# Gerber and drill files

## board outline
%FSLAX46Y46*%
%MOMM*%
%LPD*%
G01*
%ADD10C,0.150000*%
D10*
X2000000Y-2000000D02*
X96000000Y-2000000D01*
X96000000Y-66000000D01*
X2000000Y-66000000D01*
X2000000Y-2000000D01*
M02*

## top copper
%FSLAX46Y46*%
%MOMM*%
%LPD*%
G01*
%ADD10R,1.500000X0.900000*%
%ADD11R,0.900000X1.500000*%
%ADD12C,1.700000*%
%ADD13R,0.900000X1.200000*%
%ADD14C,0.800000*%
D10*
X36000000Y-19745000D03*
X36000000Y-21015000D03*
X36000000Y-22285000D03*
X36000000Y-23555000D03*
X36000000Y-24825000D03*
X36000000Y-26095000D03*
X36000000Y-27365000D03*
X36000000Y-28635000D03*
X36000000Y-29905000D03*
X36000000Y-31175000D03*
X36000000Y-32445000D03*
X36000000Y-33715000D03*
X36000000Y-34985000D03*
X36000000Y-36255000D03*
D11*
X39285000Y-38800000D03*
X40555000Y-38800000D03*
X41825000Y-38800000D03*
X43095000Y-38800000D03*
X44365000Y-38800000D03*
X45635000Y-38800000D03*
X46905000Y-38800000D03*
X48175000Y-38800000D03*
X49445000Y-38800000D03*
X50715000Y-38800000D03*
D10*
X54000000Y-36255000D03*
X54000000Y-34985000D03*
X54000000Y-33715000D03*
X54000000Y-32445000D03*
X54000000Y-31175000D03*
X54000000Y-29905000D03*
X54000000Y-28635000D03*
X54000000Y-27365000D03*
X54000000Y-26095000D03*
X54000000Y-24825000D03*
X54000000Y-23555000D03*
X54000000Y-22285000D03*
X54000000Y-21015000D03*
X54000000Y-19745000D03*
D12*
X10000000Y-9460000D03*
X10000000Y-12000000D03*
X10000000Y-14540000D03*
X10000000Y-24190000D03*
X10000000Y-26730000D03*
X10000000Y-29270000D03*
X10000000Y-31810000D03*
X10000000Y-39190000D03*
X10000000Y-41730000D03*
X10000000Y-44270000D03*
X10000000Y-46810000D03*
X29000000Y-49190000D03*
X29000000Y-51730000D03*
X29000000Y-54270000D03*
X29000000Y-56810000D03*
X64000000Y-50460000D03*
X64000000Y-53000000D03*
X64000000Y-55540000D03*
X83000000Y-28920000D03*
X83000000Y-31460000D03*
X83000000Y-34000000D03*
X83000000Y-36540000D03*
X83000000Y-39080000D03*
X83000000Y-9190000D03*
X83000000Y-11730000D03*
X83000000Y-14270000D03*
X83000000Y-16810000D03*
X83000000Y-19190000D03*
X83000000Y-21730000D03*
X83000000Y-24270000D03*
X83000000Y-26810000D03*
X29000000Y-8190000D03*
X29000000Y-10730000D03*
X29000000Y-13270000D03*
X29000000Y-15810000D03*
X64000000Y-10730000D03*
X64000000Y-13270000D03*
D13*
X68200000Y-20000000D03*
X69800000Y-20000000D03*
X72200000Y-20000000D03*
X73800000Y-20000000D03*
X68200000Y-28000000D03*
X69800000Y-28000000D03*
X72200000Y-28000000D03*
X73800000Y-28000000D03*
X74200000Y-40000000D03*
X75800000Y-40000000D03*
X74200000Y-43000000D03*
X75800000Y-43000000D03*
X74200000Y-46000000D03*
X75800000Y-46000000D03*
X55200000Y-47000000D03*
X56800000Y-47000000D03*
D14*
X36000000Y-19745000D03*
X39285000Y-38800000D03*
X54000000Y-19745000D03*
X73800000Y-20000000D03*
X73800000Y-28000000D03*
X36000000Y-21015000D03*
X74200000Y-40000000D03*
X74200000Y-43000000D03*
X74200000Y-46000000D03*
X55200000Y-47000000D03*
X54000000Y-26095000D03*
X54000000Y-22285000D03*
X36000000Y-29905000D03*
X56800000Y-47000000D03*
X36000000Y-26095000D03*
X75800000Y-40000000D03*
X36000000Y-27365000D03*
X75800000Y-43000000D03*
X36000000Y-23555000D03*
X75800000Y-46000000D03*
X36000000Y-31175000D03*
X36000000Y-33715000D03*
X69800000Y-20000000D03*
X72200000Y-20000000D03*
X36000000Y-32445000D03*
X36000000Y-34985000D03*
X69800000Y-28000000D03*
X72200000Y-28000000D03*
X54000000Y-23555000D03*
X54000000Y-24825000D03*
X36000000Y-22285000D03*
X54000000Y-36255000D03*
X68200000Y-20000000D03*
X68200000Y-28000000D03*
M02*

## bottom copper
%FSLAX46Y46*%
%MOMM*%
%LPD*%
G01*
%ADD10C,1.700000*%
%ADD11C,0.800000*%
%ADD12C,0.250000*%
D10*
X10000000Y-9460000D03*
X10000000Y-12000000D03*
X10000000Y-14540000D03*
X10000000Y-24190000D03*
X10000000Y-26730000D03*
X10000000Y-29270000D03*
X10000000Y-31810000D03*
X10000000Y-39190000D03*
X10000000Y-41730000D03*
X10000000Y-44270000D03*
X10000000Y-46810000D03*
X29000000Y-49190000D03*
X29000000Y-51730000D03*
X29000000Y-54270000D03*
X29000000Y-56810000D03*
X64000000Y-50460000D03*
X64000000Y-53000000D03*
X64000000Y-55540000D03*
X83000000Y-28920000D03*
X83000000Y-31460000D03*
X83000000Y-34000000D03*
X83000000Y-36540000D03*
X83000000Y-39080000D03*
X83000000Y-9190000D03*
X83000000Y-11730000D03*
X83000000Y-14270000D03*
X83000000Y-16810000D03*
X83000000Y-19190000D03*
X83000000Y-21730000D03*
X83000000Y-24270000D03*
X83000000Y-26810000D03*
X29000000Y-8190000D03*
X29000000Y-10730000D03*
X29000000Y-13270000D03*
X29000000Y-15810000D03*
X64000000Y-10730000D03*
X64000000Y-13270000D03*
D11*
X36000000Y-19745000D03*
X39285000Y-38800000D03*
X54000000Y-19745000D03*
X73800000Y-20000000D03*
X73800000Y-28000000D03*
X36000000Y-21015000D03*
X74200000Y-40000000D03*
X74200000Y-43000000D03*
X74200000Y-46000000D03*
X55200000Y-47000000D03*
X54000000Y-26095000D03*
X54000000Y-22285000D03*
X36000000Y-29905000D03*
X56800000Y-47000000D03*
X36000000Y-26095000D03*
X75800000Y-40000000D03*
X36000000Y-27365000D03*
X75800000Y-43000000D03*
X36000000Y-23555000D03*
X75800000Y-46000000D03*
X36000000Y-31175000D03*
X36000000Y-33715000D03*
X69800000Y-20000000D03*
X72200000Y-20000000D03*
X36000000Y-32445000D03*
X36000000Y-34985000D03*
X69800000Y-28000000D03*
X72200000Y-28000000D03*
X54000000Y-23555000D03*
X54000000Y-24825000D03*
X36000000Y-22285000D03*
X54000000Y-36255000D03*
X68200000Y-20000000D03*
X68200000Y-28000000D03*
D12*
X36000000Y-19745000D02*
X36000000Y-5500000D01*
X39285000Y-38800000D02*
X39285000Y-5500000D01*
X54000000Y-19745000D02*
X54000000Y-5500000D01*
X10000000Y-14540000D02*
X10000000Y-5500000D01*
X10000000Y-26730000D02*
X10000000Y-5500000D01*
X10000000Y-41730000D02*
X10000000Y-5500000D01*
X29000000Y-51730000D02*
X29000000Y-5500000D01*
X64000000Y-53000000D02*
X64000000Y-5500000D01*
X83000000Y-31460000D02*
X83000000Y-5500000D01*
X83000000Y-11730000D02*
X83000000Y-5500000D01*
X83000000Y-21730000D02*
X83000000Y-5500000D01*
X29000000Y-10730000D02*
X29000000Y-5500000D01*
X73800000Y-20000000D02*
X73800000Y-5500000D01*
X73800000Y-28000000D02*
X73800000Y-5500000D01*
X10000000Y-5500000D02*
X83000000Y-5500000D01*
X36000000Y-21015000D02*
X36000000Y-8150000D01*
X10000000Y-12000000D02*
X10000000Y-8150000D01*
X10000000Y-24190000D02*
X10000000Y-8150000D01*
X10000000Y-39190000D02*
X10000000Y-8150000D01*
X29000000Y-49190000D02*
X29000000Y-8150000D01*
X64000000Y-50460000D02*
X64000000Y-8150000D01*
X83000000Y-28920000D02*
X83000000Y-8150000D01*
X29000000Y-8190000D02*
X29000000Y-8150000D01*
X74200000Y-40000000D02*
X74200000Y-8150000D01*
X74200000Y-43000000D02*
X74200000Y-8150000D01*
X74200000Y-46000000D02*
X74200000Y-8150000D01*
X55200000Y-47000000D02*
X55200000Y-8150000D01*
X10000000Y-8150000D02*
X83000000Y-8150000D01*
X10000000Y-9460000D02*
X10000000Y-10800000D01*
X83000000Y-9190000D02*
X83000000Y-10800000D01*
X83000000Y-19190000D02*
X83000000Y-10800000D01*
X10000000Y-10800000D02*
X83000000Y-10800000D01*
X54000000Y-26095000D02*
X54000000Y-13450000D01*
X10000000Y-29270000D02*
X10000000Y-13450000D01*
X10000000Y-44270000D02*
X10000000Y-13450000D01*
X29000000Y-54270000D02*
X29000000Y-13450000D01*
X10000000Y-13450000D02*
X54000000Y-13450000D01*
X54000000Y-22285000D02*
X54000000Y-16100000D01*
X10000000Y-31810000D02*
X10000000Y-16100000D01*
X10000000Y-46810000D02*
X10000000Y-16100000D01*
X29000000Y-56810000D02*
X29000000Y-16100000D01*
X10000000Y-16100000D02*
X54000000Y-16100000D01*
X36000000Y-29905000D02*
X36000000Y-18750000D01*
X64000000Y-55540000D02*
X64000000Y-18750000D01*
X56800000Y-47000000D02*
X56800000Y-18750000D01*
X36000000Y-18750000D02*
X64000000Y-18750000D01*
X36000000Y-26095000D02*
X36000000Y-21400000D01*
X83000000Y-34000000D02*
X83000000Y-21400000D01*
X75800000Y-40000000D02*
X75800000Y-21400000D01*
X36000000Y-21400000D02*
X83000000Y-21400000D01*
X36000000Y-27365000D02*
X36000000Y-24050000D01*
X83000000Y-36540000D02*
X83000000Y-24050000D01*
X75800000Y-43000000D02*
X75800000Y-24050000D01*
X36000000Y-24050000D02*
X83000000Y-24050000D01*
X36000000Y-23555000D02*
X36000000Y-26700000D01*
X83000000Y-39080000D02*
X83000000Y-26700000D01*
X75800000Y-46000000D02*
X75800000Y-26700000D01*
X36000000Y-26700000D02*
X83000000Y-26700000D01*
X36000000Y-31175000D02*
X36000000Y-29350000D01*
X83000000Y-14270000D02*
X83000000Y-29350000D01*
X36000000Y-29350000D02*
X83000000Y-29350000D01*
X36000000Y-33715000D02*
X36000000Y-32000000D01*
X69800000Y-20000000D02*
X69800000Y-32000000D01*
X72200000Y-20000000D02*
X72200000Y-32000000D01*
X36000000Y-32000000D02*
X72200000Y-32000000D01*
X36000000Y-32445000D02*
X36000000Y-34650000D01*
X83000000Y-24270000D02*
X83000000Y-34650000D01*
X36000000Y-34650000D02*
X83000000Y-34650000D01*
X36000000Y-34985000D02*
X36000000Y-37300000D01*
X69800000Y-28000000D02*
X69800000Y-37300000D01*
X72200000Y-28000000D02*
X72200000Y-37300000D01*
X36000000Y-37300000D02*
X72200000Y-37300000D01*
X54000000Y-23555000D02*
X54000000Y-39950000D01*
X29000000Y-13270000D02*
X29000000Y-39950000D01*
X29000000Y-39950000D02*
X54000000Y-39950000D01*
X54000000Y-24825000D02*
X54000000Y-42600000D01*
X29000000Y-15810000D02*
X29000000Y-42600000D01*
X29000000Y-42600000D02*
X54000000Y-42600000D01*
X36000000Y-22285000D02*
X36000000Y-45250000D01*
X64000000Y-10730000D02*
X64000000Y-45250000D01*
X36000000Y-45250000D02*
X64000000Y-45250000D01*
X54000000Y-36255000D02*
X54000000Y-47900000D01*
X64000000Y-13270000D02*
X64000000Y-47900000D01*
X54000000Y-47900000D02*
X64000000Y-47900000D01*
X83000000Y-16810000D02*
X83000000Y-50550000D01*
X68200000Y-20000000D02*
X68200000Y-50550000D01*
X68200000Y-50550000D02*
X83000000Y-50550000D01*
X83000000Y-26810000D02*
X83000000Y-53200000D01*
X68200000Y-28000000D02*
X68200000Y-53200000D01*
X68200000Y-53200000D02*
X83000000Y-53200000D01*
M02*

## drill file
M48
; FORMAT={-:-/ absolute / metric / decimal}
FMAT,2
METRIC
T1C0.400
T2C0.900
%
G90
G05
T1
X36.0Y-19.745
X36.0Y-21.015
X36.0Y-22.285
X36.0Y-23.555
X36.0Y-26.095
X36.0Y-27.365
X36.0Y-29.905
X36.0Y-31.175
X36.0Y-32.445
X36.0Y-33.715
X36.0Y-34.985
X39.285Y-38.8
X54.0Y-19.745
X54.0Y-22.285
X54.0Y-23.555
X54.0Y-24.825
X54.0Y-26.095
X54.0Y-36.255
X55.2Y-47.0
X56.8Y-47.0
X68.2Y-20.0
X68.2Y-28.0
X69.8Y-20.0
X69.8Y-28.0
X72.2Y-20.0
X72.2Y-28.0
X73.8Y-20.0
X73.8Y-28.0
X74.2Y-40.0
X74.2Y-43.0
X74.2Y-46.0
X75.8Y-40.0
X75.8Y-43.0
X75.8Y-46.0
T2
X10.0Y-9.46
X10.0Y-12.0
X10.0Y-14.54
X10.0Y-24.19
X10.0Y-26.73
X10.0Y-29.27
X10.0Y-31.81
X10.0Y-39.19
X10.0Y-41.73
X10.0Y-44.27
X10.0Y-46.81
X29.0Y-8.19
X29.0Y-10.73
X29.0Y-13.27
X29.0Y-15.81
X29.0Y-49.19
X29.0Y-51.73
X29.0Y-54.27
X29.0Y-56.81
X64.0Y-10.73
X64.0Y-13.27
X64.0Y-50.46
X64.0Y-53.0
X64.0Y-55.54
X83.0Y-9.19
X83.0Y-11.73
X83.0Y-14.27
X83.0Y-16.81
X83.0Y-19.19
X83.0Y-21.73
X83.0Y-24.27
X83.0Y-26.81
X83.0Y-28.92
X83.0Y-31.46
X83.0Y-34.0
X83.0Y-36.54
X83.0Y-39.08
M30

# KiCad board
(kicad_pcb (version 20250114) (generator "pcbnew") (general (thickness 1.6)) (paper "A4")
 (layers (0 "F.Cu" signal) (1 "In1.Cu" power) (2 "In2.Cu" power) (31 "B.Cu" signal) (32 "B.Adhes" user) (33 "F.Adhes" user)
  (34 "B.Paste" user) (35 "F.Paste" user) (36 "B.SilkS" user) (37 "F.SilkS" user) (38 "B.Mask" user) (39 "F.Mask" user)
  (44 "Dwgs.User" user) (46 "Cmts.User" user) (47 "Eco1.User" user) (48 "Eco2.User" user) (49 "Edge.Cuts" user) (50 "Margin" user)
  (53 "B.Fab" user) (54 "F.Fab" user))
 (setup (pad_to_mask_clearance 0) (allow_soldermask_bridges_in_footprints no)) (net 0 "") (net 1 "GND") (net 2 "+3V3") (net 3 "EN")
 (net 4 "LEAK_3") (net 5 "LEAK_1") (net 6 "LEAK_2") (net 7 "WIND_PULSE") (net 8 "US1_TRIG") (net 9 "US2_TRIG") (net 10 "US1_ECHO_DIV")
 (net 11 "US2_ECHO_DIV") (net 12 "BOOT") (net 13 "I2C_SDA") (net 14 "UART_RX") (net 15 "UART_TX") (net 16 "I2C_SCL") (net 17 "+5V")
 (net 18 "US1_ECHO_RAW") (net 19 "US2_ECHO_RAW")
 (gr_rect (start 2 2) (end 96 66) (stroke (width 0.15) (type default)) (fill none) (layer "Edge.Cuts"))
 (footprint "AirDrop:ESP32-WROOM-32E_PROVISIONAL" (layer "F.Cu") (at 45 28)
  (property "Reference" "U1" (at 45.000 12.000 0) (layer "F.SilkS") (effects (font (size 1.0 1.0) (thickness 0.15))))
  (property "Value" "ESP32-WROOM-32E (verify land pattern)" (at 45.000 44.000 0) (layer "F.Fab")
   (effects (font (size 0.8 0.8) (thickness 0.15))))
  (pad "1" smd rect (at -9.000 -8.255) (size 1.5 0.9) (layers "F.Cu" "F.Paste" "F.Mask") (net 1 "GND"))
  (pad "2" smd rect (at -9.000 -6.985) (size 1.5 0.9) (layers "F.Cu" "F.Paste" "F.Mask") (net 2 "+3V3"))
  (pad "3" smd rect (at -9.000 -5.715) (size 1.5 0.9) (layers "F.Cu" "F.Paste" "F.Mask") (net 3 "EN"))
  (pad "4" smd rect (at -9.000 -4.445) (size 1.5 0.9) (layers "F.Cu" "F.Paste" "F.Mask") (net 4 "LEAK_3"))
  (pad "5" smd rect (at -9.000 -3.175) (size 1.5 0.9) (layers "F.Cu" "F.Paste" "F.Mask"))
  (pad "6" smd rect (at -9.000 -1.905) (size 1.5 0.9) (layers "F.Cu" "F.Paste" "F.Mask") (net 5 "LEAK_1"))
  (pad "7" smd rect (at -9.000 -0.635) (size 1.5 0.9) (layers "F.Cu" "F.Paste" "F.Mask") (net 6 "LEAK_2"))
  (pad "8" smd rect (at -9.000 0.635) (size 1.5 0.9) (layers "F.Cu" "F.Paste" "F.Mask"))
  (pad "9" smd rect (at -9.000 1.905) (size 1.5 0.9) (layers "F.Cu" "F.Paste" "F.Mask") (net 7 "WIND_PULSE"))
  (pad "10" smd rect (at -9.000 3.175) (size 1.5 0.9) (layers "F.Cu" "F.Paste" "F.Mask") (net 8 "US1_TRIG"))
  (pad "11" smd rect (at -9.000 4.445) (size 1.5 0.9) (layers "F.Cu" "F.Paste" "F.Mask") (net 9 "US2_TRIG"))
  (pad "12" smd rect (at -9.000 5.715) (size 1.5 0.9) (layers "F.Cu" "F.Paste" "F.Mask") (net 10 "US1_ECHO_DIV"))
  (pad "13" smd rect (at -9.000 6.985) (size 1.5 0.9) (layers "F.Cu" "F.Paste" "F.Mask") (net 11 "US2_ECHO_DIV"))
  (pad "14" smd rect (at -9.000 8.255) (size 1.5 0.9) (layers "F.Cu" "F.Paste" "F.Mask"))
  (pad "15" smd rect (at -5.715 10.800) (size 0.9 1.5) (layers "F.Cu" "F.Paste" "F.Mask") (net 1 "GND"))
  (pad "16" smd rect (at -4.445 10.800) (size 0.9 1.5) (layers "F.Cu" "F.Paste" "F.Mask"))
  (pad "17" smd rect (at -3.175 10.800) (size 0.9 1.5) (layers "F.Cu" "F.Paste" "F.Mask"))
  (pad "18" smd rect (at -1.905 10.800) (size 0.9 1.5) (layers "F.Cu" "F.Paste" "F.Mask"))
  (pad "19" smd rect (at -0.635 10.800) (size 0.9 1.5) (layers "F.Cu" "F.Paste" "F.Mask"))
  (pad "20" smd rect (at 0.635 10.800) (size 0.9 1.5) (layers "F.Cu" "F.Paste" "F.Mask"))
  (pad "21" smd rect (at 1.905 10.800) (size 0.9 1.5) (layers "F.Cu" "F.Paste" "F.Mask"))
  (pad "22" smd rect (at 3.175 10.800) (size 0.9 1.5) (layers "F.Cu" "F.Paste" "F.Mask"))
  (pad "23" smd rect (at 4.445 10.800) (size 0.9 1.5) (layers "F.Cu" "F.Paste" "F.Mask"))
  (pad "24" smd rect (at 5.715 10.800) (size 0.9 1.5) (layers "F.Cu" "F.Paste" "F.Mask"))
  (pad "25" smd rect (at 9.000 8.255) (size 1.5 0.9) (layers "F.Cu" "F.Paste" "F.Mask") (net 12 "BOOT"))
  (pad "26" smd rect (at 9.000 6.985) (size 1.5 0.9) (layers "F.Cu" "F.Paste" "F.Mask"))
  (pad "27" smd rect (at 9.000 5.715) (size 1.5 0.9) (layers "F.Cu" "F.Paste" "F.Mask"))
  (pad "28" smd rect (at 9.000 4.445) (size 1.5 0.9) (layers "F.Cu" "F.Paste" "F.Mask"))
  (pad "29" smd rect (at 9.000 3.175) (size 1.5 0.9) (layers "F.Cu" "F.Paste" "F.Mask"))
  (pad "30" smd rect (at 9.000 1.905) (size 1.5 0.9) (layers "F.Cu" "F.Paste" "F.Mask"))
  (pad "31" smd rect (at 9.000 0.635) (size 1.5 0.9) (layers "F.Cu" "F.Paste" "F.Mask"))
  (pad "32" smd rect (at 9.000 -0.635) (size 1.5 0.9) (layers "F.Cu" "F.Paste" "F.Mask"))
  (pad "33" smd rect (at 9.000 -1.905) (size 1.5 0.9) (layers "F.Cu" "F.Paste" "F.Mask") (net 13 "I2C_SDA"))
  (pad "34" smd rect (at 9.000 -3.175) (size 1.5 0.9) (layers "F.Cu" "F.Paste" "F.Mask") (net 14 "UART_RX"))
  (pad "35" smd rect (at 9.000 -4.445) (size 1.5 0.9) (layers "F.Cu" "F.Paste" "F.Mask") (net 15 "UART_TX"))
  (pad "36" smd rect (at 9.000 -5.715) (size 1.5 0.9) (layers "F.Cu" "F.Paste" "F.Mask") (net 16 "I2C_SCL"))
  (pad "37" smd rect (at 9.000 -6.985) (size 1.5 0.9) (layers "F.Cu" "F.Paste" "F.Mask"))
  (pad "38" smd rect (at 9.000 -8.255) (size 1.5 0.9) (layers "F.Cu" "F.Paste" "F.Mask") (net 1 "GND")))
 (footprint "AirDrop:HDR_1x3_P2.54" (layer "F.Cu") (at 10 12 0)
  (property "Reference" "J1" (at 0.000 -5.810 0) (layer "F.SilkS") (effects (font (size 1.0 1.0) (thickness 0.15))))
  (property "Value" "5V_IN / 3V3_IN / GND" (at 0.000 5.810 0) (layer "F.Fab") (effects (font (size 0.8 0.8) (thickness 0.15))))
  (pad "1" thru_hole circle (at 0.000 -2.540) (size 1.7 1.7) (drill 0.9) (layers "*.Cu" "*.Mask") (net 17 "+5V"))
  (pad "2" thru_hole circle (at 0.000 0.000) (size 1.7 1.7) (drill 0.9) (layers "*.Cu" "*.Mask") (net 2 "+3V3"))
  (pad "3" thru_hole circle (at 0.000 2.540) (size 1.7 1.7) (drill 0.9) (layers "*.Cu" "*.Mask") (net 1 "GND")))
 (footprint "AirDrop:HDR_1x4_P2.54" (layer "F.Cu") (at 10 28 0)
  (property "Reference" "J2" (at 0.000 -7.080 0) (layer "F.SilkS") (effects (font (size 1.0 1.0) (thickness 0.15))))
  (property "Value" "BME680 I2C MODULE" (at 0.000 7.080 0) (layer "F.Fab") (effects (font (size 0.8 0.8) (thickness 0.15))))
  (pad "1" thru_hole circle (at 0.000 -3.810) (size 1.7 1.7) (drill 0.9) (layers "*.Cu" "*.Mask") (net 2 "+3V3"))
  (pad "2" thru_hole circle (at 0.000 -1.270) (size 1.7 1.7) (drill 0.9) (layers "*.Cu" "*.Mask") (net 1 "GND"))
  (pad "3" thru_hole circle (at 0.000 1.270) (size 1.7 1.7) (drill 0.9) (layers "*.Cu" "*.Mask") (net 13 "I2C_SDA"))
  (pad "4" thru_hole circle (at 0.000 3.810) (size 1.7 1.7) (drill 0.9) (layers "*.Cu" "*.Mask") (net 16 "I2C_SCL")))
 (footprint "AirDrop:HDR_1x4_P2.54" (layer "F.Cu") (at 10 43 0)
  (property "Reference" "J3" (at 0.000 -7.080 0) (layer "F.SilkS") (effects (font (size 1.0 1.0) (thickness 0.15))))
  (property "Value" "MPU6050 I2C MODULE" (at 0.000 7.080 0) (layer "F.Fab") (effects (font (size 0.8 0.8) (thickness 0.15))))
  (pad "1" thru_hole circle (at 0.000 -3.810) (size 1.7 1.7) (drill 0.9) (layers "*.Cu" "*.Mask") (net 2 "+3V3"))
  (pad "2" thru_hole circle (at 0.000 -1.270) (size 1.7 1.7) (drill 0.9) (layers "*.Cu" "*.Mask") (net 1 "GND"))
  (pad "3" thru_hole circle (at 0.000 1.270) (size 1.7 1.7) (drill 0.9) (layers "*.Cu" "*.Mask") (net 13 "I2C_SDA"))
  (pad "4" thru_hole circle (at 0.000 3.810) (size 1.7 1.7) (drill 0.9) (layers "*.Cu" "*.Mask") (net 16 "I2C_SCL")))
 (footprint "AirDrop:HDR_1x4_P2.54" (layer "F.Cu") (at 29 53 0)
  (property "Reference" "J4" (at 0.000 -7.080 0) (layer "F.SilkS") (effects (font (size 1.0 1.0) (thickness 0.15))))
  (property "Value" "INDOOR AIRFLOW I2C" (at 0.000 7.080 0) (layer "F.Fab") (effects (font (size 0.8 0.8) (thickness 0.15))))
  (pad "1" thru_hole circle (at 0.000 -3.810) (size 1.7 1.7) (drill 0.9) (layers "*.Cu" "*.Mask") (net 2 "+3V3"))
  (pad "2" thru_hole circle (at 0.000 -1.270) (size 1.7 1.7) (drill 0.9) (layers "*.Cu" "*.Mask") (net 1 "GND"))
  (pad "3" thru_hole circle (at 0.000 1.270) (size 1.7 1.7) (drill 0.9) (layers "*.Cu" "*.Mask") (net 13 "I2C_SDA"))
  (pad "4" thru_hole circle (at 0.000 3.810) (size 1.7 1.7) (drill 0.9) (layers "*.Cu" "*.Mask") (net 16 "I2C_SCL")))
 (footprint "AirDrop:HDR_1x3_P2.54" (layer "F.Cu") (at 64 53 0)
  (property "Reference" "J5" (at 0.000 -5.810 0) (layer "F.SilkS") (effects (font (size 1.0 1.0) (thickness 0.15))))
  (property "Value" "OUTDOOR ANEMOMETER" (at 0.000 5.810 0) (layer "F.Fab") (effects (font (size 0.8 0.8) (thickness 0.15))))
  (pad "1" thru_hole circle (at 0.000 -2.540) (size 1.7 1.7) (drill 0.9) (layers "*.Cu" "*.Mask") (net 2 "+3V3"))
  (pad "2" thru_hole circle (at 0.000 0.000) (size 1.7 1.7) (drill 0.9) (layers "*.Cu" "*.Mask") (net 1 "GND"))
  (pad "3" thru_hole circle (at 0.000 2.540) (size 1.7 1.7) (drill 0.9) (layers "*.Cu" "*.Mask") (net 7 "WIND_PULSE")))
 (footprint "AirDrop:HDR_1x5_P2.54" (layer "F.Cu") (at 83 34 0)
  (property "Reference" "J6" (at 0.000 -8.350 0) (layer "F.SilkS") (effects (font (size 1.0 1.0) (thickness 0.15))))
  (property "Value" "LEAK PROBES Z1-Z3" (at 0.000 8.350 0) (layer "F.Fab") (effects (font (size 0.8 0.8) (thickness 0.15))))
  (pad "1" thru_hole circle (at 0.000 -5.080) (size 1.7 1.7) (drill 0.9) (layers "*.Cu" "*.Mask") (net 2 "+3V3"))
  (pad "2" thru_hole circle (at 0.000 -2.540) (size 1.7 1.7) (drill 0.9) (layers "*.Cu" "*.Mask") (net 1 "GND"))
  (pad "3" thru_hole circle (at 0.000 0.000) (size 1.7 1.7) (drill 0.9) (layers "*.Cu" "*.Mask") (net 5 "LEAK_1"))
  (pad "4" thru_hole circle (at 0.000 2.540) (size 1.7 1.7) (drill 0.9) (layers "*.Cu" "*.Mask") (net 6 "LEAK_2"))
  (pad "5" thru_hole circle (at 0.000 5.080) (size 1.7 1.7) (drill 0.9) (layers "*.Cu" "*.Mask") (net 4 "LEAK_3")))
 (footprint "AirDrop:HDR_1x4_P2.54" (layer "F.Cu") (at 83 13 0)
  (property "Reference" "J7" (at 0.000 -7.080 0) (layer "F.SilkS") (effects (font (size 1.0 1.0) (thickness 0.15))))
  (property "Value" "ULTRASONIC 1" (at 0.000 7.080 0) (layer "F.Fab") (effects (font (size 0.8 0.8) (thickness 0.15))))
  (pad "1" thru_hole circle (at 0.000 -3.810) (size 1.7 1.7) (drill 0.9) (layers "*.Cu" "*.Mask") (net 17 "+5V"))
  (pad "2" thru_hole circle (at 0.000 -1.270) (size 1.7 1.7) (drill 0.9) (layers "*.Cu" "*.Mask") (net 1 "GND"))
  (pad "3" thru_hole circle (at 0.000 1.270) (size 1.7 1.7) (drill 0.9) (layers "*.Cu" "*.Mask") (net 8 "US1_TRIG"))
  (pad "4" thru_hole circle (at 0.000 3.810) (size 1.7 1.7) (drill 0.9) (layers "*.Cu" "*.Mask") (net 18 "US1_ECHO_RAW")))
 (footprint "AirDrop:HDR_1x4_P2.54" (layer "F.Cu") (at 83 23 0)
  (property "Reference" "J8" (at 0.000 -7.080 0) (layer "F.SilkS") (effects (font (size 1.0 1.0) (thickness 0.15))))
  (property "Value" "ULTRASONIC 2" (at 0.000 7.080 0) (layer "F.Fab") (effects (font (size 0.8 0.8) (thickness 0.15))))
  (pad "1" thru_hole circle (at 0.000 -3.810) (size 1.7 1.7) (drill 0.9) (layers "*.Cu" "*.Mask") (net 17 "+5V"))
  (pad "2" thru_hole circle (at 0.000 -1.270) (size 1.7 1.7) (drill 0.9) (layers "*.Cu" "*.Mask") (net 1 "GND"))
  (pad "3" thru_hole circle (at 0.000 1.270) (size 1.7 1.7) (drill 0.9) (layers "*.Cu" "*.Mask") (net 9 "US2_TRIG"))
  (pad "4" thru_hole circle (at 0.000 3.810) (size 1.7 1.7) (drill 0.9) (layers "*.Cu" "*.Mask") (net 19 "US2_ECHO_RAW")))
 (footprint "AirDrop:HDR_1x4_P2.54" (layer "F.Cu") (at 29 12 0)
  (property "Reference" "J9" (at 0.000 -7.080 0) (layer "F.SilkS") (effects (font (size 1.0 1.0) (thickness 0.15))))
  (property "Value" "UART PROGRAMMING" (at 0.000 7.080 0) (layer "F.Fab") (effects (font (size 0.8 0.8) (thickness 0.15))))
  (pad "1" thru_hole circle (at 0.000 -3.810) (size 1.7 1.7) (drill 0.9) (layers "*.Cu" "*.Mask") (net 2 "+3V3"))
  (pad "2" thru_hole circle (at 0.000 -1.270) (size 1.7 1.7) (drill 0.9) (layers "*.Cu" "*.Mask") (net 1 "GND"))
  (pad "3" thru_hole circle (at 0.000 1.270) (size 1.7 1.7) (drill 0.9) (layers "*.Cu" "*.Mask") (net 15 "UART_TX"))
  (pad "4" thru_hole circle (at 0.000 3.810) (size 1.7 1.7) (drill 0.9) (layers "*.Cu" "*.Mask") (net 14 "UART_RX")))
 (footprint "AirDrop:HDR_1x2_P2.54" (layer "F.Cu") (at 64 12 0)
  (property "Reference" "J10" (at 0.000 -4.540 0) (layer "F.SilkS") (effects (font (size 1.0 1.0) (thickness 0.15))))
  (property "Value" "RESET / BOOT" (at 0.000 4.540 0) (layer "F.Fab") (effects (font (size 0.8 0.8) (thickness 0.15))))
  (pad "1" thru_hole circle (at 0.000 -1.270) (size 1.7 1.7) (drill 0.9) (layers "*.Cu" "*.Mask") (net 3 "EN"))
  (pad "2" thru_hole circle (at 0.000 1.270) (size 1.7 1.7) (drill 0.9) (layers "*.Cu" "*.Mask") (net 12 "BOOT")))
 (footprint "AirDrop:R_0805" (layer "F.Cu") (at 69 20)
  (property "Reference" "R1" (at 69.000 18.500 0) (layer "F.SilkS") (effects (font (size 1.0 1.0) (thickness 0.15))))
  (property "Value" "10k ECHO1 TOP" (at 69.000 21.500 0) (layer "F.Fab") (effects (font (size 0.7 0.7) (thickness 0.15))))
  (pad "1" smd rect (at -0.800 0.000) (size 0.9 1.2) (layers "F.Cu" "F.Paste" "F.Mask") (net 18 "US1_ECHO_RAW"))
  (pad "2" smd rect (at 0.800 0.000) (size 0.9 1.2) (layers "F.Cu" "F.Paste" "F.Mask") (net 10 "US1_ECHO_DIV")))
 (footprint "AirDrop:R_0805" (layer "F.Cu") (at 73 20)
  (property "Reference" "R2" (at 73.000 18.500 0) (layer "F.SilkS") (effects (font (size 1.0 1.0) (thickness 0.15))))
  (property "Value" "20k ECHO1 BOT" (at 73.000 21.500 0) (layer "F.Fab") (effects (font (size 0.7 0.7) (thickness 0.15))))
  (pad "1" smd rect (at -0.800 0.000) (size 0.9 1.2) (layers "F.Cu" "F.Paste" "F.Mask") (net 10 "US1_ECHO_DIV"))
  (pad "2" smd rect (at 0.800 0.000) (size 0.9 1.2) (layers "F.Cu" "F.Paste" "F.Mask") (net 1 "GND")))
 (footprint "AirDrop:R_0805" (layer "F.Cu") (at 69 28)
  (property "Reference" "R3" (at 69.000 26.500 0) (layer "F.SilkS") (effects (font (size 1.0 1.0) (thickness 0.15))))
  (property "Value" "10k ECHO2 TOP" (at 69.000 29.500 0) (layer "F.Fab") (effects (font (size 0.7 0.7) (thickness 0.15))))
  (pad "1" smd rect (at -0.800 0.000) (size 0.9 1.2) (layers "F.Cu" "F.Paste" "F.Mask") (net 19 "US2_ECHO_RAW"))
  (pad "2" smd rect (at 0.800 0.000) (size 0.9 1.2) (layers "F.Cu" "F.Paste" "F.Mask") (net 11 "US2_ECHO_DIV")))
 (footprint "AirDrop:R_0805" (layer "F.Cu") (at 73 28)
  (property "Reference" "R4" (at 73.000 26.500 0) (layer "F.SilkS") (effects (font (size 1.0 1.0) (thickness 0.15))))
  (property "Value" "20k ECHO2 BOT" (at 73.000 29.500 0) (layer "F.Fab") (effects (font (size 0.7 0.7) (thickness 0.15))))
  (pad "1" smd rect (at -0.800 0.000) (size 0.9 1.2) (layers "F.Cu" "F.Paste" "F.Mask") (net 11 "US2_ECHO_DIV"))
  (pad "2" smd rect (at 0.800 0.000) (size 0.9 1.2) (layers "F.Cu" "F.Paste" "F.Mask") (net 1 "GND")))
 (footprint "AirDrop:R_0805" (layer "F.Cu") (at 75 40)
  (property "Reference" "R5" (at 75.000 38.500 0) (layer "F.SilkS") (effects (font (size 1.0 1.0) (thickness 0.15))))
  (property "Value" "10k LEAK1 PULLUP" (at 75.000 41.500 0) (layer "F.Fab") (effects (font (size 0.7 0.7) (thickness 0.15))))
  (pad "1" smd rect (at -0.8 0) (size 0.9 1.2) (layers "F.Cu" "F.Paste" "F.Mask") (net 2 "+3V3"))
  (pad "2" smd rect (at 0.8 0) (size 0.9 1.2) (layers "F.Cu" "F.Paste" "F.Mask") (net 5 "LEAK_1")))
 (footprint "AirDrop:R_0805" (layer "F.Cu") (at 75 43)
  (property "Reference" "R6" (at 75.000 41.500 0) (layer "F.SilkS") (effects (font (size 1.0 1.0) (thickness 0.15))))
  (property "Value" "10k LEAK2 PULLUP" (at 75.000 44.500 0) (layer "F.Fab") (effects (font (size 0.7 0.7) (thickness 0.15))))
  (pad "1" smd rect (at -0.8 0) (size 0.9 1.2) (layers "F.Cu" "F.Paste" "F.Mask") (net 2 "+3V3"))
  (pad "2" smd rect (at 0.8 0) (size 0.9 1.2) (layers "F.Cu" "F.Paste" "F.Mask") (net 6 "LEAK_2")))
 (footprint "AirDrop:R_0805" (layer "F.Cu") (at 75 46)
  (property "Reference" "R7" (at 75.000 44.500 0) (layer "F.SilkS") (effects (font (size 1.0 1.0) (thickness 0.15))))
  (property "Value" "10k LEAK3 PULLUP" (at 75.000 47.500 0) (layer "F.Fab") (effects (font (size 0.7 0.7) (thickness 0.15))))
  (pad "1" smd rect (at -0.8 0) (size 0.9 1.2) (layers "F.Cu" "F.Paste" "F.Mask") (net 2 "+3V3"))
  (pad "2" smd rect (at 0.8 0) (size 0.9 1.2) (layers "F.Cu" "F.Paste" "F.Mask") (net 4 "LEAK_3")))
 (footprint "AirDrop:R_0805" (layer "F.Cu") (at 56 47)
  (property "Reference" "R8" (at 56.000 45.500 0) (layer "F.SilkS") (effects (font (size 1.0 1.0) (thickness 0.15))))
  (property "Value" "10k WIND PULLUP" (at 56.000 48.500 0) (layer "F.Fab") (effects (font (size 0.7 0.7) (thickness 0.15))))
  (pad "1" smd rect (at -0.8 0) (size 0.9 1.2) (layers "F.Cu" "F.Paste" "F.Mask") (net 2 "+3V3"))
  (pad "2" smd rect (at 0.8 0) (size 0.9 1.2) (layers "F.Cu" "F.Paste" "F.Mask") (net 7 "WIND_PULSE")))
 (via (at 36.000 19.745) (size 0.8) (drill 0.4) (layers "F.Cu" "B.Cu") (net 1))
 (via (at 39.285 38.800) (size 0.8) (drill 0.4) (layers "F.Cu" "B.Cu") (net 1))
 (via (at 54.000 19.745) (size 0.8) (drill 0.4) (layers "F.Cu" "B.Cu") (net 1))
 (via (at 73.800 20.000) (size 0.8) (drill 0.4) (layers "F.Cu" "B.Cu") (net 1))
 (via (at 73.800 28.000) (size 0.8) (drill 0.4) (layers "F.Cu" "B.Cu") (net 1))
 (via (at 36.000 21.015) (size 0.8) (drill 0.4) (layers "F.Cu" "B.Cu") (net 2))
 (via (at 74.200 40.000) (size 0.8) (drill 0.4) (layers "F.Cu" "B.Cu") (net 2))
 (via (at 74.200 43.000) (size 0.8) (drill 0.4) (layers "F.Cu" "B.Cu") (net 2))
 (via (at 74.200 46.000) (size 0.8) (drill 0.4) (layers "F.Cu" "B.Cu") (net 2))
 (via (at 55.200 47.000) (size 0.8) (drill 0.4) (layers "F.Cu" "B.Cu") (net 2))
 (via (at 54.000 26.095) (size 0.8) (drill 0.4) (layers "F.Cu" "B.Cu") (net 13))
 (via (at 54.000 22.285) (size 0.8) (drill 0.4) (layers "F.Cu" "B.Cu") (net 16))
 (via (at 36.000 29.905) (size 0.8) (drill 0.4) (layers "F.Cu" "B.Cu") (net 7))
 (via (at 56.800 47.000) (size 0.8) (drill 0.4) (layers "F.Cu" "B.Cu") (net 7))
 (via (at 36.000 26.095) (size 0.8) (drill 0.4) (layers "F.Cu" "B.Cu") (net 5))
 (via (at 75.800 40.000) (size 0.8) (drill 0.4) (layers "F.Cu" "B.Cu") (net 5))
 (via (at 36.000 27.365) (size 0.8) (drill 0.4) (layers "F.Cu" "B.Cu") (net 6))
 (via (at 75.800 43.000) (size 0.8) (drill 0.4) (layers "F.Cu" "B.Cu") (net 6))
 (via (at 36.000 23.555) (size 0.8) (drill 0.4) (layers "F.Cu" "B.Cu") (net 4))
 (via (at 75.800 46.000) (size 0.8) (drill 0.4) (layers "F.Cu" "B.Cu") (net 4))
 (via (at 36.000 31.175) (size 0.8) (drill 0.4) (layers "F.Cu" "B.Cu") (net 8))
 (via (at 36.000 33.715) (size 0.8) (drill 0.4) (layers "F.Cu" "B.Cu") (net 10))
 (via (at 69.800 20.000) (size 0.8) (drill 0.4) (layers "F.Cu" "B.Cu") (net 10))
 (via (at 72.200 20.000) (size 0.8) (drill 0.4) (layers "F.Cu" "B.Cu") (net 10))
 (via (at 36.000 32.445) (size 0.8) (drill 0.4) (layers "F.Cu" "B.Cu") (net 9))
 (via (at 36.000 34.985) (size 0.8) (drill 0.4) (layers "F.Cu" "B.Cu") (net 11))
 (via (at 69.800 28.000) (size 0.8) (drill 0.4) (layers "F.Cu" "B.Cu") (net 11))
 (via (at 72.200 28.000) (size 0.8) (drill 0.4) (layers "F.Cu" "B.Cu") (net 11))
 (via (at 54.000 23.555) (size 0.8) (drill 0.4) (layers "F.Cu" "B.Cu") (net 15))
 (via (at 54.000 24.825) (size 0.8) (drill 0.4) (layers "F.Cu" "B.Cu") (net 14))
 (via (at 36.000 22.285) (size 0.8) (drill 0.4) (layers "F.Cu" "B.Cu") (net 3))
 (via (at 54.000 36.255) (size 0.8) (drill 0.4) (layers "F.Cu" "B.Cu") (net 12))
 (via (at 68.200 20.000) (size 0.8) (drill 0.4) (layers "F.Cu" "B.Cu") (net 18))
 (via (at 68.200 28.000) (size 0.8) (drill 0.4) (layers "F.Cu" "B.Cu") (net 19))
 (segment (start 36.000 19.745) (end 36.000 5.500) (width 0.25) (layer "B.Cu") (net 1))
 (segment (start 39.285 38.800) (end 39.285 5.500) (width 0.25) (layer "B.Cu") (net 1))
 (segment (start 54.000 19.745) (end 54.000 5.500) (width 0.25) (layer "B.Cu") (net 1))
 (segment (start 10.000 14.540) (end 10.000 5.500) (width 0.25) (layer "B.Cu") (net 1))
 (segment (start 10.000 26.730) (end 10.000 5.500) (width 0.25) (layer "B.Cu") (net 1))
 (segment (start 10.000 41.730) (end 10.000 5.500) (width 0.25) (layer "B.Cu") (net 1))
 (segment (start 29.000 51.730) (end 29.000 5.500) (width 0.25) (layer "B.Cu") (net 1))
 (segment (start 64.000 53.000) (end 64.000 5.500) (width 0.25) (layer "B.Cu") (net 1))
 (segment (start 83.000 31.460) (end 83.000 5.500) (width 0.25) (layer "B.Cu") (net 1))
 (segment (start 83.000 11.730) (end 83.000 5.500) (width 0.25) (layer "B.Cu") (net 1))
 (segment (start 83.000 21.730) (end 83.000 5.500) (width 0.25) (layer "B.Cu") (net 1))
 (segment (start 29.000 10.730) (end 29.000 5.500) (width 0.25) (layer "B.Cu") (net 1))
 (segment (start 73.800 20.000) (end 73.800 5.500) (width 0.25) (layer "B.Cu") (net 1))
 (segment (start 73.800 28.000) (end 73.800 5.500) (width 0.25) (layer "B.Cu") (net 1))
 (segment (start 10.000 5.500) (end 83.000 5.500) (width 0.25) (layer "B.Cu") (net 1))
 (segment (start 36.000 21.015) (end 36.000 8.150) (width 0.25) (layer "B.Cu") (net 2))
 (segment (start 10.000 12.000) (end 10.000 8.150) (width 0.25) (layer "B.Cu") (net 2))
 (segment (start 10.000 24.190) (end 10.000 8.150) (width 0.25) (layer "B.Cu") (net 2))
 (segment (start 10.000 39.190) (end 10.000 8.150) (width 0.25) (layer "B.Cu") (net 2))
 (segment (start 29.000 49.190) (end 29.000 8.150) (width 0.25) (layer "B.Cu") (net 2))
 (segment (start 64.000 50.460) (end 64.000 8.150) (width 0.25) (layer "B.Cu") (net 2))
 (segment (start 83.000 28.920) (end 83.000 8.150) (width 0.25) (layer "B.Cu") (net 2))
 (segment (start 29.000 8.190) (end 29.000 8.150) (width 0.25) (layer "B.Cu") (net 2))
 (segment (start 74.200 40.000) (end 74.200 8.150) (width 0.25) (layer "B.Cu") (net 2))
 (segment (start 74.200 43.000) (end 74.200 8.150) (width 0.25) (layer "B.Cu") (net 2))
 (segment (start 74.200 46.000) (end 74.200 8.150) (width 0.25) (layer "B.Cu") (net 2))
 (segment (start 55.200 47.000) (end 55.200 8.150) (width 0.25) (layer "B.Cu") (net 2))
 (segment (start 10.000 8.150) (end 83.000 8.150) (width 0.25) (layer "B.Cu") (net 2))
 (segment (start 10.000 9.460) (end 10.000 10.800) (width 0.25) (layer "B.Cu") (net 17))
 (segment (start 83.000 9.190) (end 83.000 10.800) (width 0.25) (layer "B.Cu") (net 17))
 (segment (start 83.000 19.190) (end 83.000 10.800) (width 0.25) (layer "B.Cu") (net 17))
 (segment (start 10.000 10.800) (end 83.000 10.800) (width 0.25) (layer "B.Cu") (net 17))
 (segment (start 54.000 26.095) (end 54.000 13.450) (width 0.25) (layer "B.Cu") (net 13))
 (segment (start 10.000 29.270) (end 10.000 13.450) (width 0.25) (layer "B.Cu") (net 13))
 (segment (start 10.000 44.270) (end 10.000 13.450) (width 0.25) (layer "B.Cu") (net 13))
 (segment (start 29.000 54.270) (end 29.000 13.450) (width 0.25) (layer "B.Cu") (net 13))
 (segment (start 10.000 13.450) (end 54.000 13.450) (width 0.25) (layer "B.Cu") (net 13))
 (segment (start 54.000 22.285) (end 54.000 16.100) (width 0.25) (layer "B.Cu") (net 16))
 (segment (start 10.000 31.810) (end 10.000 16.100) (width 0.25) (layer "B.Cu") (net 16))
 (segment (start 10.000 46.810) (end 10.000 16.100) (width 0.25) (layer "B.Cu") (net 16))
 (segment (start 29.000 56.810) (end 29.000 16.100) (width 0.25) (layer "B.Cu") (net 16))
 (segment (start 10.000 16.100) (end 54.000 16.100) (width 0.25) (layer "B.Cu") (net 16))
 (segment (start 36.000 29.905) (end 36.000 18.750) (width 0.25) (layer "B.Cu") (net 7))
 (segment (start 64.000 55.540) (end 64.000 18.750) (width 0.25) (layer "B.Cu") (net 7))
 (segment (start 56.800 47.000) (end 56.800 18.750) (width 0.25) (layer "B.Cu") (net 7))
 (segment (start 36.000 18.750) (end 64.000 18.750) (width 0.25) (layer "B.Cu") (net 7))
 (segment (start 36.000 26.095) (end 36.000 21.400) (width 0.25) (layer "B.Cu") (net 5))
 (segment (start 83.000 34.000) (end 83.000 21.400) (width 0.25) (layer "B.Cu") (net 5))
 (segment (start 75.800 40.000) (end 75.800 21.400) (width 0.25) (layer "B.Cu") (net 5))
 (segment (start 36.000 21.400) (end 83.000 21.400) (width 0.25) (layer "B.Cu") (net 5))
 (segment (start 36.000 27.365) (end 36.000 24.050) (width 0.25) (layer "B.Cu") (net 6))
 (segment (start 83.000 36.540) (end 83.000 24.050) (width 0.25) (layer "B.Cu") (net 6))
 (segment (start 75.800 43.000) (end 75.800 24.050) (width 0.25) (layer "B.Cu") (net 6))
 (segment (start 36.000 24.050) (end 83.000 24.050) (width 0.25) (layer "B.Cu") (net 6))
 (segment (start 36.000 23.555) (end 36.000 26.700) (width 0.25) (layer "B.Cu") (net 4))
 (segment (start 83.000 39.080) (end 83.000 26.700) (width 0.25) (layer "B.Cu") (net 4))
 (segment (start 75.800 46.000) (end 75.800 26.700) (width 0.25) (layer "B.Cu") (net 4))
 (segment (start 36.000 26.700) (end 83.000 26.700) (width 0.25) (layer "B.Cu") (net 4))
 (segment (start 36.000 31.175) (end 36.000 29.350) (width 0.25) (layer "B.Cu") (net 8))
 (segment (start 83.000 14.270) (end 83.000 29.350) (width 0.25) (layer "B.Cu") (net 8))
 (segment (start 36.000 29.350) (end 83.000 29.350) (width 0.25) (layer "B.Cu") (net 8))
 (segment (start 36.000 33.715) (end 36.000 32.000) (width 0.25) (layer "B.Cu") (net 10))
 (segment (start 69.800 20.000) (end 69.800 32.000) (width 0.25) (layer "B.Cu") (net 10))
 (segment (start 72.200 20.000) (end 72.200 32.000) (width 0.25) (layer "B.Cu") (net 10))
 (segment (start 36.000 32.000) (end 72.200 32.000) (width 0.25) (layer "B.Cu") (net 10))
 (segment (start 36.000 32.445) (end 36.000 34.650) (width 0.25) (layer "B.Cu") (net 9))
 (segment (start 83.000 24.270) (end 83.000 34.650) (width 0.25) (layer "B.Cu") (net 9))
 (segment (start 36.000 34.650) (end 83.000 34.650) (width 0.25) (layer "B.Cu") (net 9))
 (segment (start 36.000 34.985) (end 36.000 37.300) (width 0.25) (layer "B.Cu") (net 11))
 (segment (start 69.800 28.000) (end 69.800 37.300) (width 0.25) (layer "B.Cu") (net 11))
 (segment (start 72.200 28.000) (end 72.200 37.300) (width 0.25) (layer "B.Cu") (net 11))
 (segment (start 36.000 37.300) (end 72.200 37.300) (width 0.25) (layer "B.Cu") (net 11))
 (segment (start 54.000 23.555) (end 54.000 39.950) (width 0.25) (layer "B.Cu") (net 15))
 (segment (start 29.000 13.270) (end 29.000 39.950) (width 0.25) (layer "B.Cu") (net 15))
 (segment (start 29.000 39.950) (end 54.000 39.950) (width 0.25) (layer "B.Cu") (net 15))
 (segment (start 54.000 24.825) (end 54.000 42.600) (width 0.25) (layer "B.Cu") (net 14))
 (segment (start 29.000 15.810) (end 29.000 42.600) (width 0.25) (layer "B.Cu") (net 14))
 (segment (start 29.000 42.600) (end 54.000 42.600) (width 0.25) (layer "B.Cu") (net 14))
 (segment (start 36.000 22.285) (end 36.000 45.250) (width 0.25) (layer "B.Cu") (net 3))
 (segment (start 64.000 10.730) (end 64.000 45.250) (width 0.25) (layer "B.Cu") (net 3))
 (segment (start 36.000 45.250) (end 64.000 45.250) (width 0.25) (layer "B.Cu") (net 3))
 (segment (start 54.000 36.255) (end 54.000 47.900) (width 0.25) (layer "B.Cu") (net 12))
 (segment (start 64.000 13.270) (end 64.000 47.900) (width 0.25) (layer "B.Cu") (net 12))
 (segment (start 54.000 47.900) (end 64.000 47.900) (width 0.25) (layer "B.Cu") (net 12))
 (segment (start 83.000 16.810) (end 83.000 50.550) (width 0.25) (layer "B.Cu") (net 18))
 (segment (start 68.200 20.000) (end 68.200 50.550) (width 0.25) (layer "B.Cu") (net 18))
 (segment (start 68.200 50.550) (end 83.000 50.550) (width 0.25) (layer "B.Cu") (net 18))
 (segment (start 83.000 26.810) (end 83.000 53.200) (width 0.25) (layer "B.Cu") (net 19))
 (segment (start 68.200 28.000) (end 68.200 53.200) (width 0.25) (layer "B.Cu") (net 19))
 (segment (start 68.200 53.200) (end 83.000 53.200) (width 0.25) (layer "B.Cu") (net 19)))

